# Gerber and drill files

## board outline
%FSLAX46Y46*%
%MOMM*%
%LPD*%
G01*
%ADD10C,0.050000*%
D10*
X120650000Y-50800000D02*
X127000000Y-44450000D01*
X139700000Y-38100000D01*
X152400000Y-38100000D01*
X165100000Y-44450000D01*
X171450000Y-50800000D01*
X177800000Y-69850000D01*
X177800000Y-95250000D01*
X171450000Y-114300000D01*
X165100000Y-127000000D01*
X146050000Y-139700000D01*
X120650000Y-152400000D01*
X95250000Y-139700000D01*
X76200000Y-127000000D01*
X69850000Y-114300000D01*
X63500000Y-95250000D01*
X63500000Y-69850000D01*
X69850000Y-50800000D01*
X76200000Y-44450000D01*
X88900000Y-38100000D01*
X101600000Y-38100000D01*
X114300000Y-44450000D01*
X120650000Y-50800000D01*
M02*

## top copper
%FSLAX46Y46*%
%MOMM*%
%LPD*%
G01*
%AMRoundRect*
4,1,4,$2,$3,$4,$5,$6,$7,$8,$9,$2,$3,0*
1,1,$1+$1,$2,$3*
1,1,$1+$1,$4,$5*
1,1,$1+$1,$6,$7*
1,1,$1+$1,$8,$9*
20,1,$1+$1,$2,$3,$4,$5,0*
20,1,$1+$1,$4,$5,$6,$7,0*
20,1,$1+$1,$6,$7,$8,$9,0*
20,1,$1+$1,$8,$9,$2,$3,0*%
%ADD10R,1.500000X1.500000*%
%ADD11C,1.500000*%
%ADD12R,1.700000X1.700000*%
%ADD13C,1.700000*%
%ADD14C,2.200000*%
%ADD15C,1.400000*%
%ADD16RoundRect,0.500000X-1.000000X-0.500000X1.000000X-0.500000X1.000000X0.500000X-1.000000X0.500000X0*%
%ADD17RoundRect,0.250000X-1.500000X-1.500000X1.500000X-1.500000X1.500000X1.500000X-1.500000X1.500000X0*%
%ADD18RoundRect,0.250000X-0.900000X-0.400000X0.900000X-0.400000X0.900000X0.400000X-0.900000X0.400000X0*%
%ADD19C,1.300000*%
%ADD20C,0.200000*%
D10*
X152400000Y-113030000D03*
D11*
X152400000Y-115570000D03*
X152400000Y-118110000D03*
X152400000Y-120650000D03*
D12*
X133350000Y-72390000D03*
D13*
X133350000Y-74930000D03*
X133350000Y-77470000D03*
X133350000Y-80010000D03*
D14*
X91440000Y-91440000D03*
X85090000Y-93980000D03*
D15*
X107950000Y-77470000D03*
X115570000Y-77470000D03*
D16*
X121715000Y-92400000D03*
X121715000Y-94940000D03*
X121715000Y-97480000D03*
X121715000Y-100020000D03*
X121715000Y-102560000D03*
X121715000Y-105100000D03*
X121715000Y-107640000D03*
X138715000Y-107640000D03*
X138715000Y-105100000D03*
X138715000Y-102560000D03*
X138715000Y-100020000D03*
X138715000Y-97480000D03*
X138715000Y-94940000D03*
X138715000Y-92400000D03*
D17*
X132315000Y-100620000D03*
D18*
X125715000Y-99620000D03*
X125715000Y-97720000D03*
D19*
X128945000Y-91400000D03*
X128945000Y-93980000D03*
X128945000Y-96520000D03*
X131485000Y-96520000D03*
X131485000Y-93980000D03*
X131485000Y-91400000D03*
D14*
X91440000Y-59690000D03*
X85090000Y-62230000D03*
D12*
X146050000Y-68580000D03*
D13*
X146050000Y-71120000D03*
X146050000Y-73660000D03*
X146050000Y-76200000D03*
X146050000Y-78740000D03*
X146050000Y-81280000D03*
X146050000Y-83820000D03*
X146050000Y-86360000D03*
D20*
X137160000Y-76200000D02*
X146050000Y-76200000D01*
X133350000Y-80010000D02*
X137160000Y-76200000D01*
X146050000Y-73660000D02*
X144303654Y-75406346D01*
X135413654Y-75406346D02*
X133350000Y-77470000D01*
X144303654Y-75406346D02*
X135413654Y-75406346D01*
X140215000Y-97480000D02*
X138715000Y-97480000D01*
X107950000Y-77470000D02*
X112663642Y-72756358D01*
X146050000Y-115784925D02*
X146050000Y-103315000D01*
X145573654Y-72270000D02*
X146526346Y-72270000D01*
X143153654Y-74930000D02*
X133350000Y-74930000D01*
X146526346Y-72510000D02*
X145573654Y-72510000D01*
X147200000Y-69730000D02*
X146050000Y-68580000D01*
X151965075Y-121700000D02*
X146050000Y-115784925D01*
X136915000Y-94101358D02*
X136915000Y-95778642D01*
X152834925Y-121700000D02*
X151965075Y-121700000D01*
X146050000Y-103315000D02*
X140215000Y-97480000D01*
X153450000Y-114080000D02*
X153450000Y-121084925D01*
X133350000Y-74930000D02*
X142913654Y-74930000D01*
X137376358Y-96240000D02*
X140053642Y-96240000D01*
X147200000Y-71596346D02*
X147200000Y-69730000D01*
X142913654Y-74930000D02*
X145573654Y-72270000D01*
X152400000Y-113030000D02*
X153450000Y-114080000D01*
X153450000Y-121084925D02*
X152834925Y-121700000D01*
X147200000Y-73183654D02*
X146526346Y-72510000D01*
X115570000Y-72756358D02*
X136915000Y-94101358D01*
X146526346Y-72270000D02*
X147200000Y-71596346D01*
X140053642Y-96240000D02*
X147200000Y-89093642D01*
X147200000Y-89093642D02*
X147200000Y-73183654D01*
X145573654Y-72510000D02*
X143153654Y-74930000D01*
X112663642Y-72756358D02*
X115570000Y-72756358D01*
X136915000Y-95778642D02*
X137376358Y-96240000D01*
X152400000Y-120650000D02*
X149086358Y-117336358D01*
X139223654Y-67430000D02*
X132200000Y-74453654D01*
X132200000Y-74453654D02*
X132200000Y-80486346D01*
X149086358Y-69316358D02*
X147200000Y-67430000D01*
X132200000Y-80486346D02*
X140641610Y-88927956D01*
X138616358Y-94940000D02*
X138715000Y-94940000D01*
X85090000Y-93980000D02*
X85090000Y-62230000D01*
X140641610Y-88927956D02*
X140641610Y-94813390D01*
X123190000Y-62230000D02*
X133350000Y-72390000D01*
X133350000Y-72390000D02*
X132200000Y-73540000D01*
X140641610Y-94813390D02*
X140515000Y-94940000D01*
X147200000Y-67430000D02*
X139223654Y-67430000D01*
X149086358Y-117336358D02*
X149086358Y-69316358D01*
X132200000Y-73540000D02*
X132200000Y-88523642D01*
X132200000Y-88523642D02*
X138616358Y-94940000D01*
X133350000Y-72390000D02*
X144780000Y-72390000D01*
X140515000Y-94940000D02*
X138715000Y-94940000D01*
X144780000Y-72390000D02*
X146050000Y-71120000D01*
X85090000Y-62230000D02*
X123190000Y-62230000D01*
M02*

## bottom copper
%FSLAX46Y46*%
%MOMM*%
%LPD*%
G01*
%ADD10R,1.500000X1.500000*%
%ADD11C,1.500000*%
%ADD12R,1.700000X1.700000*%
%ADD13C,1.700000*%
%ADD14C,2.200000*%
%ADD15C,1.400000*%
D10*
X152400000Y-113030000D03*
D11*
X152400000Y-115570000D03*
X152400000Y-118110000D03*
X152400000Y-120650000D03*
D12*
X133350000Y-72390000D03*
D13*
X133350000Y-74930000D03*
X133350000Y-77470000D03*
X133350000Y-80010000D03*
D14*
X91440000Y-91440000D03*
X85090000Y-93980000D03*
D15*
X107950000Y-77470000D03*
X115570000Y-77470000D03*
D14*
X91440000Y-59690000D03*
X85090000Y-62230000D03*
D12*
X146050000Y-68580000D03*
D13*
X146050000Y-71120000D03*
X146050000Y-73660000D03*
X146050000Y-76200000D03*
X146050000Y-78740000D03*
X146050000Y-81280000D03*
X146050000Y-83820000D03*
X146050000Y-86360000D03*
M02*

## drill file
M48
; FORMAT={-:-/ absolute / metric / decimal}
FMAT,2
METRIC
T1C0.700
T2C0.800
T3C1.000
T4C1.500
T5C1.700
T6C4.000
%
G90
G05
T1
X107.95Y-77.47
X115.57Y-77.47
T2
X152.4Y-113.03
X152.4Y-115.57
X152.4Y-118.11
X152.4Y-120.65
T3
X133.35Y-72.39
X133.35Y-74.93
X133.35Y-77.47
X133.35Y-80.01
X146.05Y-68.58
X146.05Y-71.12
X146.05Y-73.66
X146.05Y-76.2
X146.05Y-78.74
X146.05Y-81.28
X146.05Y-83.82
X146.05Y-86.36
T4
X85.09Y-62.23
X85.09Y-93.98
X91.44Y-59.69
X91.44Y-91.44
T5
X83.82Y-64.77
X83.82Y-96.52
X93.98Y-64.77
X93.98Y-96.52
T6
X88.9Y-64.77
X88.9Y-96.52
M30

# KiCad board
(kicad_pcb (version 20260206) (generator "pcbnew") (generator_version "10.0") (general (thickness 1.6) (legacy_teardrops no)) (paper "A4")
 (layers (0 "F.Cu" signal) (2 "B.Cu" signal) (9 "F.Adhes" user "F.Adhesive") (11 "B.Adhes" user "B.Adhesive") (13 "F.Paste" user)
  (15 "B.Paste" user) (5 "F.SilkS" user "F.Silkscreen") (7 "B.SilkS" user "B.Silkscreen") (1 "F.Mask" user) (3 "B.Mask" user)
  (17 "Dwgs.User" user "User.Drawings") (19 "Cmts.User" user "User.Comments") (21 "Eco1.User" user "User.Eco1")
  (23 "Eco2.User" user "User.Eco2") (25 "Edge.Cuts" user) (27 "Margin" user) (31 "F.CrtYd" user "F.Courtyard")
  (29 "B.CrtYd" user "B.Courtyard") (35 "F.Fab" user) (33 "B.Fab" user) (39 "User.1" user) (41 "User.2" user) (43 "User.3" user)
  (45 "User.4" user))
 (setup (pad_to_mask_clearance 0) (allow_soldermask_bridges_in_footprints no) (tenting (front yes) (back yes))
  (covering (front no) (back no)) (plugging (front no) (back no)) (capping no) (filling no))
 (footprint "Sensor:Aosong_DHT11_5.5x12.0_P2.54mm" (layer "F.Cu") (at 152.4 113.03)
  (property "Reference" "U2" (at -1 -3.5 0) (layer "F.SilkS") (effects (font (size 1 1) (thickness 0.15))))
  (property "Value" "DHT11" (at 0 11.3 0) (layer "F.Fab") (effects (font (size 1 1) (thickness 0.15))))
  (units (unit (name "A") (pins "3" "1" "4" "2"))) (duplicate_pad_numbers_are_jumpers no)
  (pad "1" thru_hole rect (at 0 0) (size 1.5 1.5) (drill 0.8) (layers "*.Cu" "*.Mask") (remove_unused_layers no) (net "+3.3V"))
  (pad "2" thru_hole circle (at 0 2.54) (size 1.5 1.5) (drill 0.8) (layers "*.Cu" "*.Mask") (remove_unused_layers no) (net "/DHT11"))
  (pad "3" thru_hole circle (at 0 5.08) (size 1.5 1.5) (drill 0.8) (layers "*.Cu" "*.Mask") (remove_unused_layers no)
   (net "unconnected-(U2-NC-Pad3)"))
  (pad "4" thru_hole circle (at 0 7.62) (size 1.5 1.5) (drill 0.8) (layers "*.Cu" "*.Mask") (remove_unused_layers no) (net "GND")))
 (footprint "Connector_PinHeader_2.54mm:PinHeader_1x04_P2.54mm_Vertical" (layer "F.Cu") (at 133.35 72.39)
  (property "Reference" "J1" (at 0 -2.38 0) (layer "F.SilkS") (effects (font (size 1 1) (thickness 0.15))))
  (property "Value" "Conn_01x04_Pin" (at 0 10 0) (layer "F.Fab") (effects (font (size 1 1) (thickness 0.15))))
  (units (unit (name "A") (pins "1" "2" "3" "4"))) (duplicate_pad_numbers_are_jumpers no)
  (pad "1" thru_hole rect (at 0 0) (size 1.7 1.7) (drill 1) (layers "*.Cu" "*.Mask") (remove_unused_layers no) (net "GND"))
  (pad "2" thru_hole circle (at 0 2.54) (size 1.7 1.7) (drill 1) (layers "*.Cu" "*.Mask") (remove_unused_layers no) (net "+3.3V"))
  (pad "3" thru_hole circle (at 0 5.08) (size 1.7 1.7) (drill 1) (layers "*.Cu" "*.Mask") (remove_unused_layers no) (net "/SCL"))
  (pad "4" thru_hole circle (at 0 7.62) (size 1.7 1.7) (drill 1) (layers "*.Cu" "*.Mask") (remove_unused_layers no) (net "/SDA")))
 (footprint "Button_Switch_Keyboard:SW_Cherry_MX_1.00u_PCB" (layer "F.Cu") (at 91.44 91.44)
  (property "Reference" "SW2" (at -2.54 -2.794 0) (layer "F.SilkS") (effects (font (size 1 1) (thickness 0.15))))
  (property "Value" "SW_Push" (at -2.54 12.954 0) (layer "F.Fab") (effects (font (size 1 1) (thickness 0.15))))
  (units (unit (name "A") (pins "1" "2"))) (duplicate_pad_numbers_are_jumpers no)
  (pad "" np_thru_hole circle (at -7.62 5.08) (size 1.7 1.7) (drill 1.7) (layers "*.Cu" "*.Mask"))
  (pad "" np_thru_hole circle (at -2.54 5.08) (size 4 4) (drill 4) (layers "*.Cu" "*.Mask"))
  (pad "" np_thru_hole circle (at 2.54 5.08) (size 1.7 1.7) (drill 1.7) (layers "*.Cu" "*.Mask"))
  (pad "1" thru_hole circle (at 0 0) (size 2.2 2.2) (drill 1.5) (layers "*.Cu" "*.Mask") (remove_unused_layers no) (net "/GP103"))
  (pad "2" thru_hole circle (at -6.35 2.54) (size 2.2 2.2) (drill 1.5) (layers "*.Cu" "*.Mask") (remove_unused_layers no) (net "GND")))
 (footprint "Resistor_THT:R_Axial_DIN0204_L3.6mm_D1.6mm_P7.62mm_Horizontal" (layer "F.Cu") (at 107.95 77.47)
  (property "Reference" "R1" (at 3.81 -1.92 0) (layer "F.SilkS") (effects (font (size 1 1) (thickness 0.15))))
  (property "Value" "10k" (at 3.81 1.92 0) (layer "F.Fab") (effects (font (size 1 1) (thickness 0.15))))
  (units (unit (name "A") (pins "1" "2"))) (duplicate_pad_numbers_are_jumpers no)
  (pad "1" thru_hole circle (at 0 0) (size 1.4 1.4) (drill 0.7) (layers "*.Cu" "*.Mask") (remove_unused_layers no) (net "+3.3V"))
  (pad "2" thru_hole circle (at 7.62 0) (size 1.4 1.4) (drill 0.7) (layers "*.Cu" "*.Mask") (remove_unused_layers no) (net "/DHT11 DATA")))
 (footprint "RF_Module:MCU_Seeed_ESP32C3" (layer "F.Cu") (at 130.215 100.02)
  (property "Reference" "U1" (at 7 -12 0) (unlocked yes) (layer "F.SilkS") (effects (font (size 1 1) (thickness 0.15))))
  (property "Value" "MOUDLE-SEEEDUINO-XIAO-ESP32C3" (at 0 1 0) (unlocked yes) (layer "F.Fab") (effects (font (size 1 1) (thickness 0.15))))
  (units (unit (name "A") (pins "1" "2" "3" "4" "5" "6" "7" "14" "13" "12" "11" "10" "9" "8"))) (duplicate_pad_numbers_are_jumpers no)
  (pad "" smd roundrect (at 1.1 -0.4) (size 1.5 1.5) (layers "F.Paste") (roundrect_rratio 0.1666666667))
  (pad "" smd roundrect (at 1.1 1.6) (size 1.5 1.5) (layers "F.Paste") (roundrect_rratio 0.1666666667))
  (pad "" smd roundrect (at 3.1 -0.4) (size 1.5 1.5) (layers "F.Paste") (roundrect_rratio 0.1666666667))
  (pad "" smd roundrect (at 3.1 1.6) (size 1.5 1.5) (layers "F.Paste") (roundrect_rratio 0.1666666667))
  (pad "1" smd roundrect (at -8.5 -7.62) (size 3 2) (layers "F.Cu" "F.Mask" "F.Paste") (roundrect_rratio 0.25)
   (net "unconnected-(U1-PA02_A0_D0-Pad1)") (thermal_bridge_angle 45))
  (pad "2" smd roundrect (at -8.5 -5.08) (size 3 2) (layers "F.Cu" "F.Mask" "F.Paste") (roundrect_rratio 0.25)
   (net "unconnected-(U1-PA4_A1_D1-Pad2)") (thermal_bridge_angle 45))
  (pad "3" smd roundrect (at -8.5 -2.54) (size 3 2) (layers "F.Cu" "F.Mask" "F.Paste") (roundrect_rratio 0.25)
   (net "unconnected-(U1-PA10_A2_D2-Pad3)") (thermal_bridge_angle 45))
  (pad "4" smd roundrect (at -8.5 0) (size 3 2) (layers "F.Cu" "F.Mask" "F.Paste") (roundrect_rratio 0.25)
   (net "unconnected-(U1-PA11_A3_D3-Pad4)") (thermal_bridge_angle 45))
  (pad "5" smd roundrect (at -8.5 2.54) (size 3 2) (layers "F.Cu" "F.Mask" "F.Paste") (roundrect_rratio 0.25)
   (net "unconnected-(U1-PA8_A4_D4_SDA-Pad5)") (thermal_bridge_angle 45))
  (pad "6" smd roundrect (at -8.5 5.08) (size 3 2) (layers "F.Cu" "F.Mask" "F.Paste") (roundrect_rratio 0.25)
   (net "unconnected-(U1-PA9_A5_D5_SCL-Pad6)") (thermal_bridge_angle 45))
  (pad "7" smd roundrect (at -8.5 7.62) (size 3 2) (layers "F.Cu" "F.Mask" "F.Paste") (roundrect_rratio 0.25)
   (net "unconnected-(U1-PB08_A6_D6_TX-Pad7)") (thermal_bridge_angle 45))
  (pad "8" smd roundrect (at 8.5 7.62) (size 3 2) (layers "F.Cu" "F.Mask" "F.Paste") (roundrect_rratio 0.25)
   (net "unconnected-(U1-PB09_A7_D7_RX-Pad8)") (thermal_bridge_angle 45))
  (pad "9" smd roundrect (at 8.5 5.08) (size 3 2) (layers "F.Cu" "F.Mask" "F.Paste") (roundrect_rratio 0.25)
   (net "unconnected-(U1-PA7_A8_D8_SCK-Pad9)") (thermal_bridge_angle 45))
  (pad "10" smd roundrect (at 8.5 2.54) (size 3 2) (layers "F.Cu" "F.Mask" "F.Paste") (roundrect_rratio 0.25)
   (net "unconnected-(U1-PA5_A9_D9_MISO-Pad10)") (thermal_bridge_angle 45))
  (pad "11" smd roundrect (at 8.5 0) (size 3 2) (layers "F.Cu" "F.Mask" "F.Paste") (roundrect_rratio 0.25)
   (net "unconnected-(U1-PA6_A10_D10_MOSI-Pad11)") (thermal_bridge_angle 45))
  (pad "12" smd roundrect (at 8.5 -2.54) (size 3 2) (layers "F.Cu" "F.Mask" "F.Paste") (roundrect_rratio 0.25) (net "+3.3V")
   (thermal_bridge_angle 45))
  (pad "13" smd roundrect (at 8.5 -5.08) (size 3 2) (layers "F.Cu" "F.Mask" "F.Paste") (roundrect_rratio 0.25) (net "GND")
   (thermal_bridge_angle 45))
  (pad "14" smd roundrect (at 8.5 -7.62) (size 3 2) (layers "F.Cu" "F.Mask" "F.Paste") (roundrect_rratio 0.25) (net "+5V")
   (thermal_bridge_angle 45))
  (pad "15" smd roundrect (at 2.1 0.6) (size 3.5 3.5) (layers "F.Cu" "F.Mask") (roundrect_rratio 0.07142857143))
  (pad "16" smd roundrect (at -4.5 -0.4) (size 2.3 1.3) (layers "F.Cu" "F.Mask" "F.Paste") (roundrect_rratio 0.1923076923))
  (pad "17" smd roundrect (at -4.5 -2.3) (size 2.3 1.3) (layers "F.Cu" "F.Mask" "F.Paste") (roundrect_rratio 0.1923076923))
  (pad "18" smd circle (at -1.27 -8.62) (size 1.3 1.3) (layers "F.Cu" "F.Mask" "F.Paste"))
  (pad "19" smd circle (at -1.27 -6.04) (size 1.3 1.3) (layers "F.Cu" "F.Mask" "F.Paste"))
  (pad "20" smd circle (at -1.27 -3.5) (size 1.3 1.3) (layers "F.Cu" "F.Mask" "F.Paste"))
  (pad "21" smd circle (at 1.27 -3.5) (size 1.3 1.3) (layers "F.Cu" "F.Mask" "F.Paste"))
  (pad "22" smd circle (at 1.27 -6.04) (size 1.3 1.3) (layers "F.Cu" "F.Mask" "F.Paste"))
  (pad "23" smd circle (at 1.27 -8.62) (size 1.3 1.3) (layers "F.Cu" "F.Mask" "F.Paste")))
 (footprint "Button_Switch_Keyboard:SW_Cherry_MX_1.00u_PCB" (layer "F.Cu") (at 91.44 59.69)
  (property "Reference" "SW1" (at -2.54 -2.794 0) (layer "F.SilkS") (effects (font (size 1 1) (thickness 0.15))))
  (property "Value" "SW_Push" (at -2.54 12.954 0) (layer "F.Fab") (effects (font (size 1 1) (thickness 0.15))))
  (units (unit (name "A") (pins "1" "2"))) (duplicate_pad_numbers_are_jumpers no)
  (pad "" np_thru_hole circle (at -7.62 5.08) (size 1.7 1.7) (drill 1.7) (layers "*.Cu" "*.Mask"))
  (pad "" np_thru_hole circle (at -2.54 5.08) (size 4 4) (drill 4) (layers "*.Cu" "*.Mask"))
  (pad "" np_thru_hole circle (at 2.54 5.08) (size 1.7 1.7) (drill 1.7) (layers "*.Cu" "*.Mask"))
  (pad "1" thru_hole circle (at 0 0) (size 2.2 2.2) (drill 1.5) (layers "*.Cu" "*.Mask") (remove_unused_layers no) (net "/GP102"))
  (pad "2" thru_hole circle (at -6.35 2.54) (size 2.2 2.2) (drill 1.5) (layers "*.Cu" "*.Mask") (remove_unused_layers no) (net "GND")))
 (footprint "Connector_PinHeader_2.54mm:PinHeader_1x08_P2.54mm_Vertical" (layer "F.Cu") (at 146.05 68.58)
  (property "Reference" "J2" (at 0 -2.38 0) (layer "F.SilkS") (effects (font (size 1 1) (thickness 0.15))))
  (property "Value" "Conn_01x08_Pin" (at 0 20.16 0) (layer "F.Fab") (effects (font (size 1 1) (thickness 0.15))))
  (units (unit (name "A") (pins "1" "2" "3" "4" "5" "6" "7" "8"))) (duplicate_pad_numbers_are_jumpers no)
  (pad "1" thru_hole rect (at 0 0) (size 1.7 1.7) (drill 1) (layers "*.Cu" "*.Mask") (remove_unused_layers no) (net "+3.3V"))
  (pad "2" thru_hole circle (at 0 2.54) (size 1.7 1.7) (drill 1) (layers "*.Cu" "*.Mask") (remove_unused_layers no) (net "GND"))
  (pad "3" thru_hole circle (at 0 5.08) (size 1.7 1.7) (drill 1) (layers "*.Cu" "*.Mask") (remove_unused_layers no) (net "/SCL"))
  (pad "4" thru_hole circle (at 0 7.62) (size 1.7 1.7) (drill 1) (layers "*.Cu" "*.Mask") (remove_unused_layers no) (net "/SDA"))
  (pad "5" thru_hole circle (at 0 10.16) (size 1.7 1.7) (drill 1) (layers "*.Cu" "*.Mask") (remove_unused_layers no)
   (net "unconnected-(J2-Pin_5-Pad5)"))
  (pad "6" thru_hole circle (at 0 12.7) (size 1.7 1.7) (drill 1) (layers "*.Cu" "*.Mask") (remove_unused_layers no)
   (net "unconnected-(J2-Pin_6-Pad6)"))
  (pad "7" thru_hole circle (at 0 15.24) (size 1.7 1.7) (drill 1) (layers "*.Cu" "*.Mask") (remove_unused_layers no)
   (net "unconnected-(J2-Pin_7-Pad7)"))
  (pad "8" thru_hole circle (at 0 17.78) (size 1.7 1.7) (drill 1) (layers "*.Cu" "*.Mask") (remove_unused_layers no)
   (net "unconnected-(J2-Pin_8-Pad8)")))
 (gr_poly
  (pts (xy 120.65 50.8) (xy 127 44.45) (xy 139.7 38.1) (xy 152.4 38.1) (xy 165.1 44.45) (xy 171.45 50.8) (xy 177.8 69.85) (xy 177.8 95.25)
   (xy 171.45 114.3) (xy 165.1 127) (xy 146.05 139.7) (xy 120.65 152.4) (xy 95.25 139.7) (xy 76.2 127) (xy 69.85 114.3) (xy 63.5 95.25)
   (xy 63.5 69.85) (xy 69.85 50.8) (xy 76.2 44.45) (xy 88.9 38.1) (xy 101.6 38.1) (xy 114.3 44.45))
  (stroke (width 0.05) (type solid)) (fill no) (layer "Edge.Cuts"))
 (segment (start 137.16 76.2) (end 146.05 76.2) (width 0.2) (layer "F.Cu") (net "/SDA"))
 (segment (start 133.35 80.01) (end 137.16 76.2) (width 0.2) (layer "F.Cu") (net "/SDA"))
 (segment (start 146.05 73.66) (end 144.303654 75.406346) (width 0.2) (layer "F.Cu") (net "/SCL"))
 (segment (start 135.413654 75.406346) (end 133.35 77.47) (width 0.2) (layer "F.Cu") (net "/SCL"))
 (segment (start 144.303654 75.406346) (end 135.413654 75.406346) (width 0.2) (layer "F.Cu") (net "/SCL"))
 (segment (start 140.215 97.48) (end 138.715 97.48) (width 0.2) (layer "F.Cu") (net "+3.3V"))
 (segment (start 107.95 77.47) (end 112.663642 72.756358) (width 0.2) (layer "F.Cu") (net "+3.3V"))
 (segment (start 146.05 115.784925) (end 146.05 103.315) (width 0.2) (layer "F.Cu") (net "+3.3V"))
 (segment (start 145.573654 72.27) (end 146.526346 72.27) (width 0.2) (layer "F.Cu") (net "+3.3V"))
 (segment (start 143.153654 74.93) (end 133.35 74.93) (width 0.2) (layer "F.Cu") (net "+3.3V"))
 (segment (start 146.526346 72.51) (end 145.573654 72.51) (width 0.2) (layer "F.Cu") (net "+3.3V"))
 (segment (start 147.2 69.73) (end 146.05 68.58) (width 0.2) (layer "F.Cu") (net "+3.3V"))
 (segment (start 151.965075 121.7) (end 146.05 115.784925) (width 0.2) (layer "F.Cu") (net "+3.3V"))
 (segment (start 136.915 94.101358) (end 136.915 95.778642) (width 0.2) (layer "F.Cu") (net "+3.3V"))
 (segment (start 152.834925 121.7) (end 151.965075 121.7) (width 0.2) (layer "F.Cu") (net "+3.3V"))
 (segment (start 146.05 103.315) (end 140.215 97.48) (width 0.2) (layer "F.Cu") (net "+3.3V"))
 (segment (start 153.45 114.08) (end 153.45 121.084925) (width 0.2) (layer "F.Cu") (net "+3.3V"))
 (segment (start 133.35 74.93) (end 142.913654 74.93) (width 0.2) (layer "F.Cu") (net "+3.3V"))
 (segment (start 137.376358 96.24) (end 140.053642 96.24) (width 0.2) (layer "F.Cu") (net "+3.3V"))
 (segment (start 147.2 71.596346) (end 147.2 69.73) (width 0.2) (layer "F.Cu") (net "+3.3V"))
 (segment (start 142.913654 74.93) (end 145.573654 72.27) (width 0.2) (layer "F.Cu") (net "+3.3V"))
 (segment (start 152.4 113.03) (end 153.45 114.08) (width 0.2) (layer "F.Cu") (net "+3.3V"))
 (segment (start 153.45 121.084925) (end 152.834925 121.7) (width 0.2) (layer "F.Cu") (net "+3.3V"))
 (segment (start 147.2 73.183654) (end 146.526346 72.51) (width 0.2) (layer "F.Cu") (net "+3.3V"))
 (segment (start 115.57 72.756358) (end 136.915 94.101358) (width 0.2) (layer "F.Cu") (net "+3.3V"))
 (segment (start 146.526346 72.27) (end 147.2 71.596346) (width 0.2) (layer "F.Cu") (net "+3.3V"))
 (segment (start 140.053642 96.24) (end 147.2 89.093642) (width 0.2) (layer "F.Cu") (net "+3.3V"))
 (segment (start 147.2 89.093642) (end 147.2 73.183654) (width 0.2) (layer "F.Cu") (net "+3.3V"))
 (segment (start 145.573654 72.51) (end 143.153654 74.93) (width 0.2) (layer "F.Cu") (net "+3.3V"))
 (segment (start 112.663642 72.756358) (end 115.57 72.756358) (width 0.2) (layer "F.Cu") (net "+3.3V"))
 (segment (start 136.915 95.778642) (end 137.376358 96.24) (width 0.2) (layer "F.Cu") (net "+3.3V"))
 (segment (start 152.4 120.65) (end 149.086358 117.336358) (width 0.2) (layer "F.Cu") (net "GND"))
 (segment (start 139.223654 67.43) (end 132.2 74.453654) (width 0.2) (layer "F.Cu") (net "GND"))
 (segment (start 132.2 74.453654) (end 132.2 80.486346) (width 0.2) (layer "F.Cu") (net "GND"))
 (segment (start 149.086358 69.316358) (end 147.2 67.43) (width 0.2) (layer "F.Cu") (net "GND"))
 (segment (start 132.2 80.486346) (end 140.64161 88.927956) (width 0.2) (layer "F.Cu") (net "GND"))
 (segment (start 138.616358 94.94) (end 138.715 94.94) (width 0.2) (layer "F.Cu") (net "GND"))
 (segment (start 85.09 93.98) (end 85.09 62.23) (width 0.2) (layer "F.Cu") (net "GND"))
 (segment (start 140.64161 88.927956) (end 140.64161 94.81339) (width 0.2) (layer "F.Cu") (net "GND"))
 (segment (start 123.19 62.23) (end 133.35 72.39) (width 0.2) (layer "F.Cu") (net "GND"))
 (segment (start 133.35 72.39) (end 132.2 73.54) (width 0.2) (layer "F.Cu") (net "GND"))
 (segment (start 140.64161 94.81339) (end 140.515 94.94) (width 0.2) (layer "F.Cu") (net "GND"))
 (segment (start 147.2 67.43) (end 139.223654 67.43) (width 0.2) (layer "F.Cu") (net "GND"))
 (segment (start 149.086358 117.336358) (end 149.086358 69.316358) (width 0.2) (layer "F.Cu") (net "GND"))
 (segment (start 132.2 73.54) (end 132.2 88.523642) (width 0.2) (layer "F.Cu") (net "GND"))
 (segment (start 132.2 88.523642) (end 138.616358 94.94) (width 0.2) (layer "F.Cu") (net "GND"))
 (segment (start 133.35 72.39) (end 144.78 72.39) (width 0.2) (layer "F.Cu") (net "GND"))
 (segment (start 140.515 94.94) (end 138.715 94.94) (width 0.2) (layer "F.Cu") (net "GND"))
 (segment (start 144.78 72.39) (end 146.05 71.12) (width 0.2) (layer "F.Cu") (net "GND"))
 (segment (start 85.09 62.23) (end 123.19 62.23) (width 0.2) (layer "F.Cu") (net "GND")))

